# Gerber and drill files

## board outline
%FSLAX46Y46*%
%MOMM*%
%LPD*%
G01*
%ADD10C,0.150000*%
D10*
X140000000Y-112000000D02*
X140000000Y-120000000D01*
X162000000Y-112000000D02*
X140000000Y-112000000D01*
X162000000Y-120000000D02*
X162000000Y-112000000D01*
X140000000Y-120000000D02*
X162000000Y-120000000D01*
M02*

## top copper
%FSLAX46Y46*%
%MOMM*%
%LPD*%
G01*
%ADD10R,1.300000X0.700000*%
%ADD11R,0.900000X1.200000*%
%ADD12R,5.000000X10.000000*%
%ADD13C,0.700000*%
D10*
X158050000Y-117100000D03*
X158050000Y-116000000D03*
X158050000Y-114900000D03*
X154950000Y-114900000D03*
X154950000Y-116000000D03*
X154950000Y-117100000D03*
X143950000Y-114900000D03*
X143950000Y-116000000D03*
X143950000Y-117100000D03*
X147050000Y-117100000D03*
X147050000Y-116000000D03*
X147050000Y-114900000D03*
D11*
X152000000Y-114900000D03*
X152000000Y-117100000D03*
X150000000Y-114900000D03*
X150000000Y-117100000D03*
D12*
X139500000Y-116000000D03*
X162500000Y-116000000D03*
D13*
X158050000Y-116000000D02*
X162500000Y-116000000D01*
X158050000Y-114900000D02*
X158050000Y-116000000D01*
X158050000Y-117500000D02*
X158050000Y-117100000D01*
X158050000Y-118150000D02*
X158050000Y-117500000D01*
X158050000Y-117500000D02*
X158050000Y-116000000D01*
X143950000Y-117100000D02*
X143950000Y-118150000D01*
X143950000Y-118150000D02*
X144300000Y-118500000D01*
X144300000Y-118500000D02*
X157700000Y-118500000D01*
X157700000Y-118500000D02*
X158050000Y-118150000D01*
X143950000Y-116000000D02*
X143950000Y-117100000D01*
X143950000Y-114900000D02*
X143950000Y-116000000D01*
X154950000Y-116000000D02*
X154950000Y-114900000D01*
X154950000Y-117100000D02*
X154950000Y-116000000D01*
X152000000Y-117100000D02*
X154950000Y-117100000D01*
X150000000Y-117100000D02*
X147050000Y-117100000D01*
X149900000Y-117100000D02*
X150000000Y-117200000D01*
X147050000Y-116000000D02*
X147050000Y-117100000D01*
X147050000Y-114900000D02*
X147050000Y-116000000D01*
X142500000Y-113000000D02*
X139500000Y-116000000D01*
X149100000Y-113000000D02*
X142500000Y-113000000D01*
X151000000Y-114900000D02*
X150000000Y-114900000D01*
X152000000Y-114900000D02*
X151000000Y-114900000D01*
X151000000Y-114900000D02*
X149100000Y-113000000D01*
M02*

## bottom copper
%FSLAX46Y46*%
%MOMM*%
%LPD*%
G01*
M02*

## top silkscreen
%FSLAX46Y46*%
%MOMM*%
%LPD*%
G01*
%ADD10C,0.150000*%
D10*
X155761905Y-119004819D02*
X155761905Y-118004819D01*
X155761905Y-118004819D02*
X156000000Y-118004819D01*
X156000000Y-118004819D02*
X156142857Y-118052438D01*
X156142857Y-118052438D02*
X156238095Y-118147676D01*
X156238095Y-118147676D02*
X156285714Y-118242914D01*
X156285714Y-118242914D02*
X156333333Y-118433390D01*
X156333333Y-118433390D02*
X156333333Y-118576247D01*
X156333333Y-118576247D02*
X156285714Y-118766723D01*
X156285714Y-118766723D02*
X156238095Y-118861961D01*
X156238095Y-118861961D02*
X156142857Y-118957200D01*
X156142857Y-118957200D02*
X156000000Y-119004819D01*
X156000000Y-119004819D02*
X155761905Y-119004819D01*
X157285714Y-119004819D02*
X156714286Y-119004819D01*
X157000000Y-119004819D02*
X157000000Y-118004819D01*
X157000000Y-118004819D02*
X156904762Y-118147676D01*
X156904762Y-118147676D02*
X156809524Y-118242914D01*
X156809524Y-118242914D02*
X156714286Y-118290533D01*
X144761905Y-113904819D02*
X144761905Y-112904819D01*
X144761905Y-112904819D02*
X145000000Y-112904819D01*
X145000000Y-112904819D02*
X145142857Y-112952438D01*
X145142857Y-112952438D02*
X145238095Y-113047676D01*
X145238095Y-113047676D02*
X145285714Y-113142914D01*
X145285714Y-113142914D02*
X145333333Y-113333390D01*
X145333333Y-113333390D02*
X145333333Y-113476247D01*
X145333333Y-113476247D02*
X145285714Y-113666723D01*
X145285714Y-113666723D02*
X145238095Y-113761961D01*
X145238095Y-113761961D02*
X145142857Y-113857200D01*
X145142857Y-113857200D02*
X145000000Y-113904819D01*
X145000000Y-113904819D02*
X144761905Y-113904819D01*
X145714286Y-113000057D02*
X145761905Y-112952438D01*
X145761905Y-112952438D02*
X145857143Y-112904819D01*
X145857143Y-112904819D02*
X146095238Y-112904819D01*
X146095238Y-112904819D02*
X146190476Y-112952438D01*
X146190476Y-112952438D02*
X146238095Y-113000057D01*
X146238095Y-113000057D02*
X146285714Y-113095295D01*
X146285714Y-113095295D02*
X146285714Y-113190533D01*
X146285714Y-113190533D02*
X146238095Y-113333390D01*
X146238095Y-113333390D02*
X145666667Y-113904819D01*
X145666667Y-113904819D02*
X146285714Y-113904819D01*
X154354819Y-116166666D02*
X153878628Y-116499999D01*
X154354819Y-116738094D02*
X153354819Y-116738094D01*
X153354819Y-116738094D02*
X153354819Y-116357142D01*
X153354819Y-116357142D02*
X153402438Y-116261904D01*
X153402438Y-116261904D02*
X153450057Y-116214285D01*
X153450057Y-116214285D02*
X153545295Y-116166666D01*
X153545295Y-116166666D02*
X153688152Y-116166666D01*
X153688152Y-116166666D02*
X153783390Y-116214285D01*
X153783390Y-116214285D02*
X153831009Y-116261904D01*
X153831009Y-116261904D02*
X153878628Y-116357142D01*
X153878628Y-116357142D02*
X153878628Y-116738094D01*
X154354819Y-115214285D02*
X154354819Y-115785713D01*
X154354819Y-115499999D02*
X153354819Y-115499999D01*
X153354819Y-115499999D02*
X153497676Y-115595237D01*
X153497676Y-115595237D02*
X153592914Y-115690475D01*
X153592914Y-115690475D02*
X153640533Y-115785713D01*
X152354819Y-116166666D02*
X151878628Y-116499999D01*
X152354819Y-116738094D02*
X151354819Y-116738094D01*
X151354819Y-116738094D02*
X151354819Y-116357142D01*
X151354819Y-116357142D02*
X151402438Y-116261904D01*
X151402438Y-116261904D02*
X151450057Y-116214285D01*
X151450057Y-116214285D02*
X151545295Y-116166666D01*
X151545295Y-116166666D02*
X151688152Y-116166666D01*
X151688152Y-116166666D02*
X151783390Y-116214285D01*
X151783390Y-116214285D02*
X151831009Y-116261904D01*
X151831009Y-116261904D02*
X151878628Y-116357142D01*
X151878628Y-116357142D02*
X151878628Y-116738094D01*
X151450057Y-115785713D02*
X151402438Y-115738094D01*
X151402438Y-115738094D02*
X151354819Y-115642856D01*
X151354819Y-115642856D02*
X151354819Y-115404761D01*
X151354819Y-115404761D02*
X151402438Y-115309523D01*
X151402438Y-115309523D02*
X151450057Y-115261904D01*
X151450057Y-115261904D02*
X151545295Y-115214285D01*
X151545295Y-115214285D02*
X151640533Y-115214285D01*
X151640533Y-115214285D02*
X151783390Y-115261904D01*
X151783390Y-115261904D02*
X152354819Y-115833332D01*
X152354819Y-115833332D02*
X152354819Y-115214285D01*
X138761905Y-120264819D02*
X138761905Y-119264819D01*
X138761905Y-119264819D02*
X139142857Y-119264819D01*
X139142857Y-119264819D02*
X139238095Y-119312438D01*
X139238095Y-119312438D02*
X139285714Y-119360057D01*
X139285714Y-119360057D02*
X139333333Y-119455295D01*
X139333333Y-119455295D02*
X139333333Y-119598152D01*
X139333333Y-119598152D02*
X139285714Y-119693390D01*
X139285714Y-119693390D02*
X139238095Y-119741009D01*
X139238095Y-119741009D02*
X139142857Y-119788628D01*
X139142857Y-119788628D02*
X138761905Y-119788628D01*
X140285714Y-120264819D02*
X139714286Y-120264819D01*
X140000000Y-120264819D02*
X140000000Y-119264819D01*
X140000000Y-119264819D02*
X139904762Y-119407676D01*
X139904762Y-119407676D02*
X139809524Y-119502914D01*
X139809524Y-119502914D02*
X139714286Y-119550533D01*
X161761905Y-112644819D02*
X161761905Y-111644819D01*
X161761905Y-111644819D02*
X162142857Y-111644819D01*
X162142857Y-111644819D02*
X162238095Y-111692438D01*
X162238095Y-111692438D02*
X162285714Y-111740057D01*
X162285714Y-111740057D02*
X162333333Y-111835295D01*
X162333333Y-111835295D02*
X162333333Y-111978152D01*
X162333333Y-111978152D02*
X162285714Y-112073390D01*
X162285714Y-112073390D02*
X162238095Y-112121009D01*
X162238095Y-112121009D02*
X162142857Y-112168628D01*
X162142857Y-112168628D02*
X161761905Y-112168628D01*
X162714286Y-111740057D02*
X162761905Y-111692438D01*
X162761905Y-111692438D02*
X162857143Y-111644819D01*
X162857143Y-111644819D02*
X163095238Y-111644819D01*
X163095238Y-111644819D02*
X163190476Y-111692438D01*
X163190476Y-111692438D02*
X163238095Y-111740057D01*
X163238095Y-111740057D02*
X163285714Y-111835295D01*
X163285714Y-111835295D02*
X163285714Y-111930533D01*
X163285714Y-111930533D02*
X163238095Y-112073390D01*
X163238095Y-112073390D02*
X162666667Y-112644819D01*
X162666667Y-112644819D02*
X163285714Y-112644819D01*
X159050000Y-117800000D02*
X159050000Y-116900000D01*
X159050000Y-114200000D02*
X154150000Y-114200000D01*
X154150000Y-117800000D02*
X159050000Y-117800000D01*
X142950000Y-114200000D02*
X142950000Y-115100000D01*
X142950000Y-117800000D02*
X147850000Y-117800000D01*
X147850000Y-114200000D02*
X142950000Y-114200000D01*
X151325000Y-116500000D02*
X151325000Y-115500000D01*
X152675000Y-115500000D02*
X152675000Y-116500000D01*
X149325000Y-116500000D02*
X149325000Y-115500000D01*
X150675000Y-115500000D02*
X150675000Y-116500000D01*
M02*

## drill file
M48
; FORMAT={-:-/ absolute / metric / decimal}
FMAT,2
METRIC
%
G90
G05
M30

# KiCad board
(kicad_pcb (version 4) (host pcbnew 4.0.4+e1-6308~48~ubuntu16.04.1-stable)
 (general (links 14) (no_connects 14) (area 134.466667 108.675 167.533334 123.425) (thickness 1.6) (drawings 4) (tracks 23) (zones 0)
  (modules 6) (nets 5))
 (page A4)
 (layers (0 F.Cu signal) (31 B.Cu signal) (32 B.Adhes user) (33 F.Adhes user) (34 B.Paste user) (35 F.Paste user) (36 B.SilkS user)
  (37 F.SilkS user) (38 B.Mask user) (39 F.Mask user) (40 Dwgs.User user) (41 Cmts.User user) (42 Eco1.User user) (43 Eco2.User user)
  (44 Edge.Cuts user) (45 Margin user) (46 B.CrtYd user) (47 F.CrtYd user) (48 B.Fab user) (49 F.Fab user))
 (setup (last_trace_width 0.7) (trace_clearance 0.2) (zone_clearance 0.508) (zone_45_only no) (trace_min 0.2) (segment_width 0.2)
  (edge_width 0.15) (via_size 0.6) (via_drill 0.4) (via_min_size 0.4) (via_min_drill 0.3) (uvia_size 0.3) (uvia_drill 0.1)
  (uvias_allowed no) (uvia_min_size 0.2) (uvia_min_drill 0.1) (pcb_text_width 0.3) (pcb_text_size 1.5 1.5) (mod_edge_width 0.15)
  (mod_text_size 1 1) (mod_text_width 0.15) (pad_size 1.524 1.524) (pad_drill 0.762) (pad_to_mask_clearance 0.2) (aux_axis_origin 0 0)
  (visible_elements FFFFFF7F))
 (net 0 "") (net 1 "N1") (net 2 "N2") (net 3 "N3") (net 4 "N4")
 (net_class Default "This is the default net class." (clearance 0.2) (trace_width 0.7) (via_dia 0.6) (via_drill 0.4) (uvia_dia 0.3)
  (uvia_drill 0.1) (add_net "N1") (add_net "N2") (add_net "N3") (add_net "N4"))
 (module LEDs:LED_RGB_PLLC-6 (layer F.Cu) (at 156.5 116 180)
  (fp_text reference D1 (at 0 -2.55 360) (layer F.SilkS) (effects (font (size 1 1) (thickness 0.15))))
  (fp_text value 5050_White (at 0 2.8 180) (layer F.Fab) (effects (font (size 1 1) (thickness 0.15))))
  (fp_line (start -2.55 -1.8) (end -2.55 -0.9) (layer F.SilkS) (width 0.15))
  (fp_line (start -2.55 1.8) (end 2.35 1.8) (layer F.SilkS) (width 0.15))
  (fp_line (start 2.35 -1.8) (end -2.55 -1.8) (layer F.SilkS) (width 0.15))
  (pad 1 smd rect (at -1.55 -1.1 270) (size 0.7 1.3) (layers F.Cu F.Paste F.Mask) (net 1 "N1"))
  (pad 2 smd rect (at -1.55 0 270) (size 0.7 1.3) (layers F.Cu F.Paste F.Mask) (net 1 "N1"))
  (pad 3 smd rect (at -1.55 1.1 270) (size 0.7 1.3) (layers F.Cu F.Paste F.Mask) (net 1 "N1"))
  (pad 4 smd rect (at 1.55 1.1 270) (size 0.7 1.3) (layers F.Cu F.Paste F.Mask) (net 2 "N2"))
  (pad 5 smd rect (at 1.55 0 270) (size 0.7 1.3) (layers F.Cu F.Paste F.Mask) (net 2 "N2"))
  (pad 6 smd rect (at 1.55 -1.1 270) (size 0.7 1.3) (layers F.Cu F.Paste F.Mask) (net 2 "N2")))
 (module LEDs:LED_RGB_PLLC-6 (layer F.Cu) (at 145.5 116)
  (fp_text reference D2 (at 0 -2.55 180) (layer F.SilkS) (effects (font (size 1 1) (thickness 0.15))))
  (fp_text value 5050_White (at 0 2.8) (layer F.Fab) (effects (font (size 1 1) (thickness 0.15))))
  (fp_line (start -2.55 -1.8) (end -2.55 -0.9) (layer F.SilkS) (width 0.15))
  (fp_line (start -2.55 1.8) (end 2.35 1.8) (layer F.SilkS) (width 0.15))
  (fp_line (start 2.35 -1.8) (end -2.55 -1.8) (layer F.SilkS) (width 0.15))
  (pad 1 smd rect (at -1.55 -1.1 90) (size 0.7 1.3) (layers F.Cu F.Paste F.Mask) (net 1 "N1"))
  (pad 2 smd rect (at -1.55 0 90) (size 0.7 1.3) (layers F.Cu F.Paste F.Mask) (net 1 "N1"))
  (pad 3 smd rect (at -1.55 1.1 90) (size 0.7 1.3) (layers F.Cu F.Paste F.Mask) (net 1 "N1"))
  (pad 4 smd rect (at 1.55 1.1 90) (size 0.7 1.3) (layers F.Cu F.Paste F.Mask) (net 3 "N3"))
  (pad 5 smd rect (at 1.55 0 90) (size 0.7 1.3) (layers F.Cu F.Paste F.Mask) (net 3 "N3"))
  (pad 6 smd rect (at 1.55 -1.1 90) (size 0.7 1.3) (layers F.Cu F.Paste F.Mask) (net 3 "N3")))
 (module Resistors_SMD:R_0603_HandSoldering (layer F.Cu) (at 152 116 270)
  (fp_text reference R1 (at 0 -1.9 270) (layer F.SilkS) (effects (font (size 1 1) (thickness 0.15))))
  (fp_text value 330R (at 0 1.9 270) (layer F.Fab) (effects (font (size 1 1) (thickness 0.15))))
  (fp_line (start 0.5 0.675) (end -0.5 0.675) (layer F.SilkS) (width 0.15))
  (fp_line (start -0.5 -0.675) (end 0.5 -0.675) (layer F.SilkS) (width 0.15))
  (pad 1 smd rect (at -1.1 0 270) (size 1.2 0.9) (layers F.Cu F.Paste F.Mask) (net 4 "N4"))
  (pad 2 smd rect (at 1.1 0 270) (size 1.2 0.9) (layers F.Cu F.Paste F.Mask) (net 2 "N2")))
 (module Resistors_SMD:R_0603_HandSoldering (layer F.Cu) (at 150 116 270)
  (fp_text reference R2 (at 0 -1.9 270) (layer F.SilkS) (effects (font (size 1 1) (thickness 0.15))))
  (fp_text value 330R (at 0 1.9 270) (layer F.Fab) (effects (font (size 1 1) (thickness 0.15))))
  (fp_line (start 0.5 0.675) (end -0.5 0.675) (layer F.SilkS) (width 0.15))
  (fp_line (start -0.5 -0.675) (end 0.5 -0.675) (layer F.SilkS) (width 0.15))
  (pad 1 smd rect (at -1.1 0 270) (size 1.2 0.9) (layers F.Cu F.Paste F.Mask) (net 4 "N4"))
  (pad 2 smd rect (at 1.1 0 270) (size 1.2 0.9) (layers F.Cu F.Paste F.Mask) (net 3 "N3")))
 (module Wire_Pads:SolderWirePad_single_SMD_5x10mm (layer F.Cu) (at 139.5 116 180)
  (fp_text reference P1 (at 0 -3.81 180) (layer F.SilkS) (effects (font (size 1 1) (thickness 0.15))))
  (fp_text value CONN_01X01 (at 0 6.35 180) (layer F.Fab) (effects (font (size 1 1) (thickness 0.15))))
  (pad 1 smd rect (at 0 0 180) (size 5 10) (layers F.Cu F.Paste F.Mask) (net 4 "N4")))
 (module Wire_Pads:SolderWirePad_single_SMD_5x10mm (layer F.Cu) (at 162.5 116)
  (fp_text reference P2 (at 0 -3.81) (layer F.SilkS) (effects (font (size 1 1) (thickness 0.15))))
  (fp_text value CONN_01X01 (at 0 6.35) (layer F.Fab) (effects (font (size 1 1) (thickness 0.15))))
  (pad 1 smd rect (at 0 0) (size 5 10) (layers F.Cu F.Paste F.Mask) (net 1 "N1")))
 (gr_line (start 140 112) (end 140 120) (layer Edge.Cuts) (width 0.15))
 (gr_line (start 162 112) (end 140 112) (layer Edge.Cuts) (width 0.15))
 (gr_line (start 162 120) (end 162 112) (layer Edge.Cuts) (width 0.15))
 (gr_line (start 140 120) (end 162 120) (layer Edge.Cuts) (width 0.15))
 (segment (start 158.05 116) (end 162.5 116) (width 0.7) (layer F.Cu) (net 1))
 (segment (start 158.05 114.9) (end 158.05 116) (width 0.7) (layer F.Cu) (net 1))
 (segment (start 158.05 117.5) (end 158.05 117.1) (width 0.7) (layer F.Cu) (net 1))
 (segment (start 158.05 118.15) (end 158.05 117.5) (width 0.7) (layer F.Cu) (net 1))
 (segment (start 158.05 117.5) (end 158.05 116) (width 0.7) (layer F.Cu) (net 1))
 (segment (start 143.95 117.1) (end 143.95 118.15) (width 0.7) (layer F.Cu) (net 1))
 (segment (start 143.95 118.15) (end 144.3 118.5) (width 0.7) (layer F.Cu) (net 1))
 (segment (start 144.3 118.5) (end 157.7 118.5) (width 0.7) (layer F.Cu) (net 1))
 (segment (start 157.7 118.5) (end 158.05 118.15) (width 0.7) (layer F.Cu) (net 1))
 (segment (start 143.95 116) (end 143.95 117.1) (width 0.7) (layer F.Cu) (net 1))
 (segment (start 143.95 114.9) (end 143.95 116) (width 0.7) (layer F.Cu) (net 1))
 (segment (start 154.95 116) (end 154.95 114.9) (width 0.7) (layer F.Cu) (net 2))
 (segment (start 154.95 117.1) (end 154.95 116) (width 0.7) (layer F.Cu) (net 2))
 (segment (start 152 117.1) (end 154.95 117.1) (width 0.7) (layer F.Cu) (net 2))
 (segment (start 150 117.1) (end 147.05 117.1) (width 0.7) (layer F.Cu) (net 3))
 (segment (start 149.9 117.1) (end 150 117.2) (width 0.7) (layer F.Cu) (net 3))
 (segment (start 147.05 116) (end 147.05 117.1) (width 0.7) (layer F.Cu) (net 3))
 (segment (start 147.05 114.9) (end 147.05 116) (width 0.7) (layer F.Cu) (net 3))
 (segment (start 142.5 113) (end 139.5 116) (width 0.7) (layer F.Cu) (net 4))
 (segment (start 149.1 113) (end 142.5 113) (width 0.7) (layer F.Cu) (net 4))
 (segment (start 151 114.9) (end 150 114.9) (width 0.7) (layer F.Cu) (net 4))
 (segment (start 152 114.9) (end 151 114.9) (width 0.7) (layer F.Cu) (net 4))
 (segment (start 151 114.9) (end 149.1 113) (width 0.7) (layer F.Cu) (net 4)))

